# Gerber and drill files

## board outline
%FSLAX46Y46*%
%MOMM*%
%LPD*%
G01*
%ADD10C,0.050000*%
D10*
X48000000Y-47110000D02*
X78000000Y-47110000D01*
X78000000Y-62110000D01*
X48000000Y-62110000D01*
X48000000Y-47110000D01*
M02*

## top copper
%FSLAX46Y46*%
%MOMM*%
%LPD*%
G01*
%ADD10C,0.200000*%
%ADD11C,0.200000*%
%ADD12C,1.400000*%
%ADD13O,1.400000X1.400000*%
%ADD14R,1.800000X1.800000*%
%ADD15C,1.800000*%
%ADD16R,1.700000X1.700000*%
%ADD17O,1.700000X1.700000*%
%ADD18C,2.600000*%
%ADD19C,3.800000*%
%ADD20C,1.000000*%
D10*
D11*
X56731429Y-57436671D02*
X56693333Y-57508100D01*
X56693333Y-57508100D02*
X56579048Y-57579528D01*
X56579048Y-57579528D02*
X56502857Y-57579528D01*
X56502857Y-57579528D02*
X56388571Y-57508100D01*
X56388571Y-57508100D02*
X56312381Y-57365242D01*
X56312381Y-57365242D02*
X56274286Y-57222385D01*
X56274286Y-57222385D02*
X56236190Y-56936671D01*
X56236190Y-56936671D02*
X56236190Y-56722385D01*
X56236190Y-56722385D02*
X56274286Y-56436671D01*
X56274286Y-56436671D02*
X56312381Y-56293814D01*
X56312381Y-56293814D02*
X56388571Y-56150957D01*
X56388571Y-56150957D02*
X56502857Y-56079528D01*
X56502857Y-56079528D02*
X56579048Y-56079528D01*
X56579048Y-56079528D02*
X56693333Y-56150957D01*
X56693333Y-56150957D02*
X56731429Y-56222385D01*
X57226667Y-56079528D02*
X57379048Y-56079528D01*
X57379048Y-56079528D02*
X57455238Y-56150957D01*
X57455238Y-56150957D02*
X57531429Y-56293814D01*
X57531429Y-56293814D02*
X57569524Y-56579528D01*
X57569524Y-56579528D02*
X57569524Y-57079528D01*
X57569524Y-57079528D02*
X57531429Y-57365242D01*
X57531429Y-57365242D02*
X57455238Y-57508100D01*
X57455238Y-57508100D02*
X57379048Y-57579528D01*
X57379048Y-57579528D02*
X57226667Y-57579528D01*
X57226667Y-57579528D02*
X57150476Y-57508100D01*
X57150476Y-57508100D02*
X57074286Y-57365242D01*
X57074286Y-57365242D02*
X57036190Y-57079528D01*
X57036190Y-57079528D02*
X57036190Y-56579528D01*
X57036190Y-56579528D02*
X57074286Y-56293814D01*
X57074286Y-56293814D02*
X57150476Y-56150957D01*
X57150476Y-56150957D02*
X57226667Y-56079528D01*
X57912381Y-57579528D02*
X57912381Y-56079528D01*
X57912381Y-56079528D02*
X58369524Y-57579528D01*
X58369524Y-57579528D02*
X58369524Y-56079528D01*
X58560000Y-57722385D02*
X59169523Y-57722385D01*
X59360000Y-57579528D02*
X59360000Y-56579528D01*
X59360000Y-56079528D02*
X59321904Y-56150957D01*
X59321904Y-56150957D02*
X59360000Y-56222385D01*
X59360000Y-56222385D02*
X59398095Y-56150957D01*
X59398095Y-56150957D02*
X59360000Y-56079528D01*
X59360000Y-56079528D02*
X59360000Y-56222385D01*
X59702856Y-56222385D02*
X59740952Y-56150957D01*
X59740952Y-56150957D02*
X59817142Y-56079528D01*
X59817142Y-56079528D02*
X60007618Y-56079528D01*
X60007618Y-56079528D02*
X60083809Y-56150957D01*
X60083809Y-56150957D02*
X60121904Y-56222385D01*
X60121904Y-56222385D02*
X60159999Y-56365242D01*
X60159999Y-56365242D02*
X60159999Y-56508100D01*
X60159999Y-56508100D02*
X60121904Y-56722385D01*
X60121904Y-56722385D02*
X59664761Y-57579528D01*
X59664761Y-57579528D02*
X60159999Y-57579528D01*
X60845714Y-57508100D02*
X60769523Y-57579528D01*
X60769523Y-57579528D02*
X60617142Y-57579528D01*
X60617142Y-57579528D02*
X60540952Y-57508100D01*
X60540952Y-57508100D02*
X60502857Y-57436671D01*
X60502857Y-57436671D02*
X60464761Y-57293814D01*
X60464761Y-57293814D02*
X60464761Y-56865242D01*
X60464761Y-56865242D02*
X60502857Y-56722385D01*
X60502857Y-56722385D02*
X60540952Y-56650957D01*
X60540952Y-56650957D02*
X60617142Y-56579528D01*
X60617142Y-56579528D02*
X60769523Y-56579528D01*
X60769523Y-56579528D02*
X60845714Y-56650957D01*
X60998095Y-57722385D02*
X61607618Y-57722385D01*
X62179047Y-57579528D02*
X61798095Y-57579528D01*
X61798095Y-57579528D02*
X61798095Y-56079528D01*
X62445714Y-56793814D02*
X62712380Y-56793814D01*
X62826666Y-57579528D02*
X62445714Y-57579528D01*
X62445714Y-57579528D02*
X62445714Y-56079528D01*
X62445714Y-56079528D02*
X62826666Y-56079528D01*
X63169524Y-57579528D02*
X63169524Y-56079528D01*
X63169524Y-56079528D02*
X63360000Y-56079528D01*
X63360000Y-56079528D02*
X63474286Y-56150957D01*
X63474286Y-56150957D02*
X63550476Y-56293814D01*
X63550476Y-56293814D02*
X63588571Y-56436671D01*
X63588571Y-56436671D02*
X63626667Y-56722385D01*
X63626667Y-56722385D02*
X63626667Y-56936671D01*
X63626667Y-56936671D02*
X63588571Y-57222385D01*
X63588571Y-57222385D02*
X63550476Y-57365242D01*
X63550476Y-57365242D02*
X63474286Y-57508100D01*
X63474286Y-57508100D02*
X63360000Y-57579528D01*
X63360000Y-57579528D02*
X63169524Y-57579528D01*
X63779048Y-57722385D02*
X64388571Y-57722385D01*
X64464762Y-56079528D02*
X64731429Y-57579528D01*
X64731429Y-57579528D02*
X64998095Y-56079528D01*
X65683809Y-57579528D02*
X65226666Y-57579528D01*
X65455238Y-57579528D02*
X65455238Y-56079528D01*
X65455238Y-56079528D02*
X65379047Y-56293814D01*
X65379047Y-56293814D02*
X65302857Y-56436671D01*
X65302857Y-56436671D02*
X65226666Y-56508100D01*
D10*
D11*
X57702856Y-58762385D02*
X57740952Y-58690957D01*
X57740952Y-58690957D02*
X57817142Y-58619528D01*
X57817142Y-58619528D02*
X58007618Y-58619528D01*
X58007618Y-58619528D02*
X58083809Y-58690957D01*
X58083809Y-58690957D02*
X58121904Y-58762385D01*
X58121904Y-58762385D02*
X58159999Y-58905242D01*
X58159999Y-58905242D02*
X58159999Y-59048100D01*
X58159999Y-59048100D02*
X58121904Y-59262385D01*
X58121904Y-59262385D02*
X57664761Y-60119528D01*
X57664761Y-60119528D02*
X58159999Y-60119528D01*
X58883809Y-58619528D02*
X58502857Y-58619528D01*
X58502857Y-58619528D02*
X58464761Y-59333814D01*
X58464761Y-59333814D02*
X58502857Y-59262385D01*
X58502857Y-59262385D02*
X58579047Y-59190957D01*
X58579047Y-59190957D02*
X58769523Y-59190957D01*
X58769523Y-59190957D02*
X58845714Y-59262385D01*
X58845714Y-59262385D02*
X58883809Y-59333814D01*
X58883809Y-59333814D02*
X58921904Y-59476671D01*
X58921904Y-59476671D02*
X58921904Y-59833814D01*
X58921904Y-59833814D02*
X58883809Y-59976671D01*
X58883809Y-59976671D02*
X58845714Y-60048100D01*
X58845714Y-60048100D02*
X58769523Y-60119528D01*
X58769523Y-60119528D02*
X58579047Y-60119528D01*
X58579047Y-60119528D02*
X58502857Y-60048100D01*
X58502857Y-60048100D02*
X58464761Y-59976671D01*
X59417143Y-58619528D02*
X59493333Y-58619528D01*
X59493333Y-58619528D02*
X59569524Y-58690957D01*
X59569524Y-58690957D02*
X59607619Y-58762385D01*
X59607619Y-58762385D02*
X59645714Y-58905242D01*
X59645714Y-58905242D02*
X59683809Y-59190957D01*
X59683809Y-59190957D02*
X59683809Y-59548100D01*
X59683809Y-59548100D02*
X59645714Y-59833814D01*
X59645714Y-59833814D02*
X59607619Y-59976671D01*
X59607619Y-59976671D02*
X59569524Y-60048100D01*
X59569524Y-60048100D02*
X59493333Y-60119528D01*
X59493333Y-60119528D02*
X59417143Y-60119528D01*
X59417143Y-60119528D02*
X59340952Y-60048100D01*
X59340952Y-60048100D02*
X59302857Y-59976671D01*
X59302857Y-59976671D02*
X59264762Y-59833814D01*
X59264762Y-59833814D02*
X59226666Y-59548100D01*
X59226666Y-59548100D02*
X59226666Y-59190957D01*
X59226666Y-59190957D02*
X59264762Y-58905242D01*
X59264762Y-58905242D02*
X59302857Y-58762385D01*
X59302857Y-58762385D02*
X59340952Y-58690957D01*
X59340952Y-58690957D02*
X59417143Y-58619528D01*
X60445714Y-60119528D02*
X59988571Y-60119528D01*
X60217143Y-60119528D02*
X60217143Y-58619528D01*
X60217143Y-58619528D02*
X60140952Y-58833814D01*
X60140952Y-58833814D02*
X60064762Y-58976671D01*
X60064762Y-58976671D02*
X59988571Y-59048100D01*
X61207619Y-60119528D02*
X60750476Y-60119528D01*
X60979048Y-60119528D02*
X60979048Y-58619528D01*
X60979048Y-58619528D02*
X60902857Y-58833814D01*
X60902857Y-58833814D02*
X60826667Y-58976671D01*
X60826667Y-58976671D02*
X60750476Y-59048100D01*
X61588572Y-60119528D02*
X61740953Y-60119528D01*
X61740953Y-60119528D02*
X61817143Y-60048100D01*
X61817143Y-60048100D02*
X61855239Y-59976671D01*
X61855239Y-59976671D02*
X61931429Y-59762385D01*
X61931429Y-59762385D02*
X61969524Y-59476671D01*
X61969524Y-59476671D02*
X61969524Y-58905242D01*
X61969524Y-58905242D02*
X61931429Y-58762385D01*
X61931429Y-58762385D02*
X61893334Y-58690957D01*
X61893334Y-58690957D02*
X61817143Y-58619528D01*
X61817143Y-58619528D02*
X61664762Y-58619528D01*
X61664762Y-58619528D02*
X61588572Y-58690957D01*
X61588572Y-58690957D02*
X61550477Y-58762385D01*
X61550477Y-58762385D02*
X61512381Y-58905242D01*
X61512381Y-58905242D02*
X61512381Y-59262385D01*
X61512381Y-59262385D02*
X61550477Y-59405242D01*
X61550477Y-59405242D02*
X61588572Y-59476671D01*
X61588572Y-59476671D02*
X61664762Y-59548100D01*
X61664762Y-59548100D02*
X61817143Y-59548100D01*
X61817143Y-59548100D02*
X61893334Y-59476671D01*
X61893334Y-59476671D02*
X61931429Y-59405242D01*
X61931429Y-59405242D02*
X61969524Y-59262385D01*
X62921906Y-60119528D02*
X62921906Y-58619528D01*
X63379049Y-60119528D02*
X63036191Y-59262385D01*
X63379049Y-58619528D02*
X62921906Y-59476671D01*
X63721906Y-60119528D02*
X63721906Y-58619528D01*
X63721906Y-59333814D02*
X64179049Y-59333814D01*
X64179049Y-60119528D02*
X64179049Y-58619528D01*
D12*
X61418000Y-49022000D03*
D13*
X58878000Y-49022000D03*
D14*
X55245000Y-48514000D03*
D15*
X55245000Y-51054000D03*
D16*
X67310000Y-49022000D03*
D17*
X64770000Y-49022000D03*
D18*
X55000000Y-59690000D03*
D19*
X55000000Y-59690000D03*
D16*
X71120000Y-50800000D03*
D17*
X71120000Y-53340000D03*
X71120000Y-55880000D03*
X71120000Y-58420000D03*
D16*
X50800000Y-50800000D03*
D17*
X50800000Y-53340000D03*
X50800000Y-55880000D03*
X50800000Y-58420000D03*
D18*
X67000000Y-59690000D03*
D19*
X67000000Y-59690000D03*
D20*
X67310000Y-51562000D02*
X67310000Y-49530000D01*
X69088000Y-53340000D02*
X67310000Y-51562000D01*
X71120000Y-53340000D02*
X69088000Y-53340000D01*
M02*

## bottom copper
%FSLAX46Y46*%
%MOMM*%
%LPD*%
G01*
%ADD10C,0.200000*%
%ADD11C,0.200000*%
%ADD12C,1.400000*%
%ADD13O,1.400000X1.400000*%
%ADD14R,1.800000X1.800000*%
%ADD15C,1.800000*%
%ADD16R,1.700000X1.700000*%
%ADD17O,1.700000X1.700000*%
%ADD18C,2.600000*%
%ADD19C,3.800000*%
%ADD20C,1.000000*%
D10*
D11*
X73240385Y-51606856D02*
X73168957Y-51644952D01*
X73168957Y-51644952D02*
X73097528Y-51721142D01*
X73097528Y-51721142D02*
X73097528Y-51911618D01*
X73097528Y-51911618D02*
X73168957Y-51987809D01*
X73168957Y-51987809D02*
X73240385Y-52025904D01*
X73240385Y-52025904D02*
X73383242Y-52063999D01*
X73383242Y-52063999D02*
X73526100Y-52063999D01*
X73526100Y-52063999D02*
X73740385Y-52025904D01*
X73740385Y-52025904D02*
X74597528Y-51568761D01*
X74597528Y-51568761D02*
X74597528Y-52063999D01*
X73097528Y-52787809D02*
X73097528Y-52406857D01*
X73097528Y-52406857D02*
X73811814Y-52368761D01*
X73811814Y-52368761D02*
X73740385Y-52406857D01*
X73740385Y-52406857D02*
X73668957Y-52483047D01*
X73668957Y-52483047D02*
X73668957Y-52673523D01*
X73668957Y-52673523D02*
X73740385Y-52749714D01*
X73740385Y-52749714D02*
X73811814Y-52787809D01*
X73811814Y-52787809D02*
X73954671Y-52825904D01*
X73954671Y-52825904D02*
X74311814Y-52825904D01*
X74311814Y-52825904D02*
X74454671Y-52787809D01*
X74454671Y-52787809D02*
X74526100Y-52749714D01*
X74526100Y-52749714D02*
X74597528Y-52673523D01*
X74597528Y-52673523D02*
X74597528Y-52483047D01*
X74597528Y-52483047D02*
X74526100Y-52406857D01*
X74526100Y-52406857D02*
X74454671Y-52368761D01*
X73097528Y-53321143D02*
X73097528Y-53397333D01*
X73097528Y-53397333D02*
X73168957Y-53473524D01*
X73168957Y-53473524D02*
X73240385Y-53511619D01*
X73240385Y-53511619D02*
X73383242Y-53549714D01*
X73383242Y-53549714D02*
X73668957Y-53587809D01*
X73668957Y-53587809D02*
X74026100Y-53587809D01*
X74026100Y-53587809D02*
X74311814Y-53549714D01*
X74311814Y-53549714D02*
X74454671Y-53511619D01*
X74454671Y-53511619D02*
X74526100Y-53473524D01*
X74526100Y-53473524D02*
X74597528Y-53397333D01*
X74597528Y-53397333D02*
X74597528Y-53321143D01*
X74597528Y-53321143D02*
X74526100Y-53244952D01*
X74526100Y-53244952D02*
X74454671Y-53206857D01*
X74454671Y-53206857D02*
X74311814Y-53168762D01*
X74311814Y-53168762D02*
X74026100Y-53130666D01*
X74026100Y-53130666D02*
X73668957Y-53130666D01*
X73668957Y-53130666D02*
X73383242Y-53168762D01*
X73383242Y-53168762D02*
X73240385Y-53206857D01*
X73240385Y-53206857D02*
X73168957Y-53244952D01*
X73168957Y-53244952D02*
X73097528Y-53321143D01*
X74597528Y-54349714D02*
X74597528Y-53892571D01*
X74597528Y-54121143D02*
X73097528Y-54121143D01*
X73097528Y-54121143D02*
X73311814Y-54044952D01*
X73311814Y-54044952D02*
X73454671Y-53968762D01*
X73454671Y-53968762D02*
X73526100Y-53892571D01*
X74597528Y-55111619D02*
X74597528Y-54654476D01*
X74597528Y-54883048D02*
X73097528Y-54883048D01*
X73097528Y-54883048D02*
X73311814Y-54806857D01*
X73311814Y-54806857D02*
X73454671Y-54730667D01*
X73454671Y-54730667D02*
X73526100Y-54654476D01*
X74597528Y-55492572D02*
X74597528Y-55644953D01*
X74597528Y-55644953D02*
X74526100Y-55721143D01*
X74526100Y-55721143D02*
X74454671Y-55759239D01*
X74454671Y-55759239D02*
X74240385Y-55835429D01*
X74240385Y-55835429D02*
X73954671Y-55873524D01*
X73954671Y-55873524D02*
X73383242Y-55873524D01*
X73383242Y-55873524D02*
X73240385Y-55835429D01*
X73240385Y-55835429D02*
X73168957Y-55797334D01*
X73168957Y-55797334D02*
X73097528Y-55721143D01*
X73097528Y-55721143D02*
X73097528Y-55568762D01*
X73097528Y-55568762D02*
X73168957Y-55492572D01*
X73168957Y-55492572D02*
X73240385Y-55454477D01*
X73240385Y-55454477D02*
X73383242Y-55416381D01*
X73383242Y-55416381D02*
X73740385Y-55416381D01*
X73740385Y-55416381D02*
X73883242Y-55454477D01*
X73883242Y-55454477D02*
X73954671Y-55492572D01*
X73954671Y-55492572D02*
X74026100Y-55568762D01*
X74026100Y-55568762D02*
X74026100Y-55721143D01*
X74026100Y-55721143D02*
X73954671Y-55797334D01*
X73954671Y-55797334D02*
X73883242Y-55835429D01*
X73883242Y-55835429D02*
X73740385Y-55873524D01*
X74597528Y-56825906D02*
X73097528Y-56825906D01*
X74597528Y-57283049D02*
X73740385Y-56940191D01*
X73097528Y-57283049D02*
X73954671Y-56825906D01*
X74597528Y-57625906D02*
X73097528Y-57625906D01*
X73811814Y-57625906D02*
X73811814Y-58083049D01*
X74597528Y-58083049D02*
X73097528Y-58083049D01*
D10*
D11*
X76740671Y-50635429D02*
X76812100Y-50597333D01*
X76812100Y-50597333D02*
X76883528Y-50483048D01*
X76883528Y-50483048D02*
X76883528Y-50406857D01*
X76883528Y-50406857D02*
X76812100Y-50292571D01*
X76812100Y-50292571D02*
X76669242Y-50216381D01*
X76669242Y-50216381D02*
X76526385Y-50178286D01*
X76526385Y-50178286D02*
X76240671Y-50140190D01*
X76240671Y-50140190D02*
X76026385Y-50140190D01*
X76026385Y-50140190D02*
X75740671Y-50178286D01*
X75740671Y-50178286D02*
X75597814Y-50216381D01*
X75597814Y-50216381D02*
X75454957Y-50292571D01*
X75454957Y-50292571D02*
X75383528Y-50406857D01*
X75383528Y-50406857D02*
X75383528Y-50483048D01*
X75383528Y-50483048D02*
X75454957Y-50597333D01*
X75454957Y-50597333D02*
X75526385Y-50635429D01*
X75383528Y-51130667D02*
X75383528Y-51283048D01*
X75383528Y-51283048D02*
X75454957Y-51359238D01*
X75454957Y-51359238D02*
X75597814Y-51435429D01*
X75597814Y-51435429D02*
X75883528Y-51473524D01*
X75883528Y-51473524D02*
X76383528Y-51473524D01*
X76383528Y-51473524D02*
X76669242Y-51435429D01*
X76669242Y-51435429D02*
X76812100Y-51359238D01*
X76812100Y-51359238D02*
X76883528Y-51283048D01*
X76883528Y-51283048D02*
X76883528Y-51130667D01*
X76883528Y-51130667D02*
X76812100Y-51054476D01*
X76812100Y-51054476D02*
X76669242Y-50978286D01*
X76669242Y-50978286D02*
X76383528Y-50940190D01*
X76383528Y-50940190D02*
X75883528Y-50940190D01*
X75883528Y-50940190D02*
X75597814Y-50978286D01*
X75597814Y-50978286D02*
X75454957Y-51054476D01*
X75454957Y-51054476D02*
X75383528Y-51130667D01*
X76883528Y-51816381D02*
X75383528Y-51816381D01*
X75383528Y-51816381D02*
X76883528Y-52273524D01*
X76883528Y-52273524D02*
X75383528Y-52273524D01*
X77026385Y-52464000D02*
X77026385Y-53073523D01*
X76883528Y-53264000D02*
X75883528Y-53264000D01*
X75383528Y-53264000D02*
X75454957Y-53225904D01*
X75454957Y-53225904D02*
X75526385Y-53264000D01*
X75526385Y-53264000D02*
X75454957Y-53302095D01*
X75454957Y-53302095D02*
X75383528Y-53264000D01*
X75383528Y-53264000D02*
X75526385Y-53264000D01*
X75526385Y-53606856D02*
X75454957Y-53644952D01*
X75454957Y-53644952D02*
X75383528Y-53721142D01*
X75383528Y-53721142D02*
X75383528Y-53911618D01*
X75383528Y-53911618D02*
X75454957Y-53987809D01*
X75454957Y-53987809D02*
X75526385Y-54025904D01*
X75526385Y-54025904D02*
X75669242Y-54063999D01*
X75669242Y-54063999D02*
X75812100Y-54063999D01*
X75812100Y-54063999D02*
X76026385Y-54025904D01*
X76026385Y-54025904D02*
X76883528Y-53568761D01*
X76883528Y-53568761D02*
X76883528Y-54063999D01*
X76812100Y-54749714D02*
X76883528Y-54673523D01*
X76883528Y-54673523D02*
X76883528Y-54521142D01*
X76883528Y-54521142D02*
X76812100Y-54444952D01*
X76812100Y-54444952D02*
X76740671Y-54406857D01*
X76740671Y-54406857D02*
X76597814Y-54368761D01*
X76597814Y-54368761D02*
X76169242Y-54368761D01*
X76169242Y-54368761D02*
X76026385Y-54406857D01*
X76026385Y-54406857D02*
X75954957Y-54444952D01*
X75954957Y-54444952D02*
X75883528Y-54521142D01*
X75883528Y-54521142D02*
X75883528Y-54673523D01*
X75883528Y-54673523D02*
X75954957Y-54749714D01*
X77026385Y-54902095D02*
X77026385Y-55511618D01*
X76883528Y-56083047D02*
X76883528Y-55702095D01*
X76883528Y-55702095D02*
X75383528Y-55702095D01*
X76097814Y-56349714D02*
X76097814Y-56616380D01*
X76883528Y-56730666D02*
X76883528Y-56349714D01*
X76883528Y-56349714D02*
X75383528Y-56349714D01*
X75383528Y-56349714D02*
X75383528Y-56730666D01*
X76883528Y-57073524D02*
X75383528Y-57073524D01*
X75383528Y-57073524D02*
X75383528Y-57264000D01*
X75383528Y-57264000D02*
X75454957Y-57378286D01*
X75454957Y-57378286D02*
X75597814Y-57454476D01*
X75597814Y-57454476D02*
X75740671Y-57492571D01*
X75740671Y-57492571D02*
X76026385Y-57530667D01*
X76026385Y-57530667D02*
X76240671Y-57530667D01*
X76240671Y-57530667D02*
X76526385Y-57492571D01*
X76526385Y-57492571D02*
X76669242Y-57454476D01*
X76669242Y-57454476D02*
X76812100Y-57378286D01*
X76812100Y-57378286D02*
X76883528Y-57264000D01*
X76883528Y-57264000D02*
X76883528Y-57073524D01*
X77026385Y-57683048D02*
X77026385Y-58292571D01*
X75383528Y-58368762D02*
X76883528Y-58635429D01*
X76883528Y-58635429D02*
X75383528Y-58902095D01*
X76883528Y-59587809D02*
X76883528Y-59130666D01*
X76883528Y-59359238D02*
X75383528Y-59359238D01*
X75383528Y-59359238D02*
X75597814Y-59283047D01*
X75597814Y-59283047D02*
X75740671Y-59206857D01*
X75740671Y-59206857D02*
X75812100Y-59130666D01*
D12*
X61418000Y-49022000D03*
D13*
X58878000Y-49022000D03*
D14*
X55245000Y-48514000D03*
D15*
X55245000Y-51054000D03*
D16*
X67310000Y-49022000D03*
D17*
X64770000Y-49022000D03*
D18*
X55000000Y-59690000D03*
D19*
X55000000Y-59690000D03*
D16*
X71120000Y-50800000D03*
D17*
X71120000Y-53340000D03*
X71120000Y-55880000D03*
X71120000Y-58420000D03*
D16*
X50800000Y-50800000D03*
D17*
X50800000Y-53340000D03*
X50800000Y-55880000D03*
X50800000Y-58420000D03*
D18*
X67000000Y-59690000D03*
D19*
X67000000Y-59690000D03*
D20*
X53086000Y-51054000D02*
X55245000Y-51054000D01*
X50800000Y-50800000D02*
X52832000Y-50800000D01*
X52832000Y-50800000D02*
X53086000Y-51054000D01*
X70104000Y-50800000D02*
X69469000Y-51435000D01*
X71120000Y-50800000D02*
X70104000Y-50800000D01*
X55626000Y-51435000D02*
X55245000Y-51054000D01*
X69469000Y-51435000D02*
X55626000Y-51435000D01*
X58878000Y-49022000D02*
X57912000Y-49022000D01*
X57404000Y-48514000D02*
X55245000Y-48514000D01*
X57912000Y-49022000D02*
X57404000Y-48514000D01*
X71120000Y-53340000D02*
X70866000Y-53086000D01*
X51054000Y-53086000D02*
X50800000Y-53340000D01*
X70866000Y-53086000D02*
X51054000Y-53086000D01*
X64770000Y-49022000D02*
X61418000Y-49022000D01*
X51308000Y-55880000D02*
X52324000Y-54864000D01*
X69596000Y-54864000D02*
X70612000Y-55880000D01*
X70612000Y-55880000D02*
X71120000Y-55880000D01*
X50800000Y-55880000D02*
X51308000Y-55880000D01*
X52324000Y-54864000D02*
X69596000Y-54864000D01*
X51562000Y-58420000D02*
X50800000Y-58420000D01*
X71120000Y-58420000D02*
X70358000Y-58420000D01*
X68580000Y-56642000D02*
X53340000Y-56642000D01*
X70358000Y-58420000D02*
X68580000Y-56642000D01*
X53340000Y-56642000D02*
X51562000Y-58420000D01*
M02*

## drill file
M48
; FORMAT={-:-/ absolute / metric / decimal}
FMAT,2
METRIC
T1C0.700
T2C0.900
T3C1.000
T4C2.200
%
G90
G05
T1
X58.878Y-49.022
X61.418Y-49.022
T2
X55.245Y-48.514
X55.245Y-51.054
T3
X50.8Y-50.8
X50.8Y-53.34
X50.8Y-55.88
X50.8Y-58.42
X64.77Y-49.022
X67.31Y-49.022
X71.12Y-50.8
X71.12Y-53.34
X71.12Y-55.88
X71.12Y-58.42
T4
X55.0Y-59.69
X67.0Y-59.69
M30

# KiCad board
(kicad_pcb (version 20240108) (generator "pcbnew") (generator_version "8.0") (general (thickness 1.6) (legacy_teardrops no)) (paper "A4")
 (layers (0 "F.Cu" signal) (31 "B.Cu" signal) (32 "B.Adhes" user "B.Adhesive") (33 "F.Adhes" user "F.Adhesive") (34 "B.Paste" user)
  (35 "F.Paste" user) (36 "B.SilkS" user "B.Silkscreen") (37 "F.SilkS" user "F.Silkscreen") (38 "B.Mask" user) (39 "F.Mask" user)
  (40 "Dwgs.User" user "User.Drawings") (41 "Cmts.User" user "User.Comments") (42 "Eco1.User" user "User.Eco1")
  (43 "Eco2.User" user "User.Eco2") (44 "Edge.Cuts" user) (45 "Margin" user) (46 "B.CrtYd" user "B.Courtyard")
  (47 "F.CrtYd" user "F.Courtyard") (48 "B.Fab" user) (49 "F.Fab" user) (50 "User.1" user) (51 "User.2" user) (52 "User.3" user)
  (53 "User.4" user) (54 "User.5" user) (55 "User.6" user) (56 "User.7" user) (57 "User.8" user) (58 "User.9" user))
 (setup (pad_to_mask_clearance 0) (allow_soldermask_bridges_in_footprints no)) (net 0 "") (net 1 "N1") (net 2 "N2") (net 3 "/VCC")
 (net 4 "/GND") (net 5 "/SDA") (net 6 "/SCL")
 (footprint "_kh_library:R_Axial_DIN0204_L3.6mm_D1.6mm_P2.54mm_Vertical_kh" (layer "F.Cu") (at 61.418 49.022 180)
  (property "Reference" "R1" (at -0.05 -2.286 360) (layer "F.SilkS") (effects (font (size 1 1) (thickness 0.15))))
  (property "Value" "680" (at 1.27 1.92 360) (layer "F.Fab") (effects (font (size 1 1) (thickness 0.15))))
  (pad "1" thru_hole circle (at 0 0 180) (size 1.4 1.4) (drill 0.7) (layers "*.Cu" "*.Mask") (remove_unused_layers no) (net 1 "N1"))
  (pad "2" thru_hole oval (at 2.54 0 180) (size 1.4 1.4) (drill 0.7) (layers "*.Cu" "*.Mask") (remove_unused_layers no) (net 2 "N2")))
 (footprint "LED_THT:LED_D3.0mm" (layer "F.Cu") (at 55.245 48.514 -90)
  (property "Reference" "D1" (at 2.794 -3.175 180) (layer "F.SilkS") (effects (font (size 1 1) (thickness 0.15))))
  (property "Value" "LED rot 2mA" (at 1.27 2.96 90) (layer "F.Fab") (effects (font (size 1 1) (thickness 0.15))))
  (pad "1" thru_hole rect (at 0 0 270) (size 1.8 1.8) (drill 0.9) (layers "*.Cu" "*.Mask") (remove_unused_layers no) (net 2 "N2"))
  (pad "2" thru_hole circle (at 2.54 0 270) (size 1.8 1.8) (drill 0.9) (layers "*.Cu" "*.Mask") (remove_unused_layers no) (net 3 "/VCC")))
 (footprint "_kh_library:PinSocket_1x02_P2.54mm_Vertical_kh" (layer "F.Cu") (at 67.31 49.022 -90)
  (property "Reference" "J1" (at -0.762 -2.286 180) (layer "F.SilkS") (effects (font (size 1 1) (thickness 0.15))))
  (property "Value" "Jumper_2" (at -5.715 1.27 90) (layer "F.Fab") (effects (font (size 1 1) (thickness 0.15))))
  (pad "1" thru_hole rect (at 0 0 270) (size 1.7 1.7) (drill 1) (layers "*.Cu" "*.Mask") (remove_unused_layers no) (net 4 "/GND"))
  (pad "2" thru_hole oval (at 0 2.54 270) (size 1.7 1.7) (drill 1) (layers "*.Cu" "*.Mask") (remove_unused_layers no) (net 1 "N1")))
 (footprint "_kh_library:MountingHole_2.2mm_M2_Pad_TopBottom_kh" (layer "F.Cu") (at 55 59.69)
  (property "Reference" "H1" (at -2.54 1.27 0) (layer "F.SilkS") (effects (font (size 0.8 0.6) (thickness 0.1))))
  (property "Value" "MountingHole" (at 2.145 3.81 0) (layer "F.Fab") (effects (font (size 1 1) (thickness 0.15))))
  (pad "1" thru_hole circle (at 0 0) (size 2.6 2.6) (drill 2.2) (layers "*.Cu" "*.Mask") (remove_unused_layers no))
  (pad "1" connect circle (at 0 0) (size 3.8 3.8) (layers "F.Cu" "F.Mask"))
  (pad "1" connect circle (at 0 0) (size 3.8 3.8) (layers "B.Cu" "B.Mask")))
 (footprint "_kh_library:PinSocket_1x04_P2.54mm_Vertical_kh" (layer "F.Cu") (at 71.12 50.8)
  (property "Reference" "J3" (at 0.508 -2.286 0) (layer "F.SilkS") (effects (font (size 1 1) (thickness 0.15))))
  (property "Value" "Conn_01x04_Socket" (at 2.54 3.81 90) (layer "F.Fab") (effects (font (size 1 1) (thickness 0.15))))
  (pad "1" thru_hole rect (at 0 0) (size 1.7 1.7) (drill 1) (layers "*.Cu" "*.Mask") (remove_unused_layers no) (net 3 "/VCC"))
  (pad "2" thru_hole oval (at 0 2.54) (size 1.7 1.7) (drill 1) (layers "*.Cu" "*.Mask") (remove_unused_layers no) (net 4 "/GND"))
  (pad "3" thru_hole oval (at 0 5.08) (size 1.7 1.7) (drill 1) (layers "*.Cu" "*.Mask") (remove_unused_layers no) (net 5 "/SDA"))
  (pad "4" thru_hole oval (at 0 7.62) (size 1.7 1.7) (drill 1) (layers "*.Cu" "*.Mask") (remove_unused_layers no) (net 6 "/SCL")))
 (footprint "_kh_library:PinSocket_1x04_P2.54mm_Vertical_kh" (layer "F.Cu") (at 50.8 50.8)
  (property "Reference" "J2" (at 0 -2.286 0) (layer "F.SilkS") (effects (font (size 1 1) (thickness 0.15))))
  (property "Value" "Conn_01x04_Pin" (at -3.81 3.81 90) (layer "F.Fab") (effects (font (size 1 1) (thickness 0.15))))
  (pad "1" thru_hole rect (at 0 0) (size 1.7 1.7) (drill 1) (layers "*.Cu" "*.Mask") (remove_unused_layers no) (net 3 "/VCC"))
  (pad "2" thru_hole oval (at 0 2.54) (size 1.7 1.7) (drill 1) (layers "*.Cu" "*.Mask") (remove_unused_layers no) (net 4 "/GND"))
  (pad "3" thru_hole oval (at 0 5.08) (size 1.7 1.7) (drill 1) (layers "*.Cu" "*.Mask") (remove_unused_layers no) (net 5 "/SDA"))
  (pad "4" thru_hole oval (at 0 7.62) (size 1.7 1.7) (drill 1) (layers "*.Cu" "*.Mask") (remove_unused_layers no) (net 6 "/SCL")))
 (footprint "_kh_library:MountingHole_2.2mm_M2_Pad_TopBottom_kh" (layer "F.Cu") (at 67 59.69)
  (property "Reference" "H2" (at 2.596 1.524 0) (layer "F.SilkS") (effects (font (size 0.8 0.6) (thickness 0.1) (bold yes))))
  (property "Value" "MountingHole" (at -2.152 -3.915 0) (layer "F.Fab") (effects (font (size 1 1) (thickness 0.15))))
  (pad "1" thru_hole circle (at 0 0) (size 2.6 2.6) (drill 2.2) (layers "*.Cu" "*.Mask") (remove_unused_layers no))
  (pad "1" connect circle (at 0 0) (size 3.8 3.8) (layers "F.Cu" "F.Mask"))
  (pad "1" connect circle (at 0 0) (size 3.8 3.8) (layers "B.Cu" "B.Mask")))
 (gr_rect (start 48 47.11) (end 78 62.11) (stroke (width 0.05) (type default)) (fill none) (layer "Edge.Cuts"))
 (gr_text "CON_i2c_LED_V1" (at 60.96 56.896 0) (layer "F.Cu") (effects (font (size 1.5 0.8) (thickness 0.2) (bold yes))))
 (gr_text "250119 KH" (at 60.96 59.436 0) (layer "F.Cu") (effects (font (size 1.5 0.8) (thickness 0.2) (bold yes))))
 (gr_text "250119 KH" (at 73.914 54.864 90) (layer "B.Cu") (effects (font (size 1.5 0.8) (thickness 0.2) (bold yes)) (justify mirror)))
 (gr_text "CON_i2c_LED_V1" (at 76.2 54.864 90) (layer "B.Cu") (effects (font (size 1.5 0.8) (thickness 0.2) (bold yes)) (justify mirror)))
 (segment (start 53.086 51.054) (end 55.245 51.054) (width 1) (layer "B.Cu") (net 3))
 (segment (start 50.8 50.8) (end 52.832 50.8) (width 1) (layer "B.Cu") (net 3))
 (segment (start 52.832 50.8) (end 53.086 51.054) (width 1) (layer "B.Cu") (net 3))
 (segment (start 70.104 50.8) (end 69.469 51.435) (width 1) (layer "B.Cu") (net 3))
 (segment (start 71.12 50.8) (end 70.104 50.8) (width 1) (layer "B.Cu") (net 3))
 (segment (start 55.626 51.435) (end 55.245 51.054) (width 1) (layer "B.Cu") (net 3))
 (segment (start 69.469 51.435) (end 55.626 51.435) (width 1) (layer "B.Cu") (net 3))
 (segment (start 58.878 49.022) (end 57.912 49.022) (width 1) (layer "B.Cu") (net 2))
 (segment (start 57.404 48.514) (end 55.245 48.514) (width 1) (layer "B.Cu") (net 2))
 (segment (start 57.912 49.022) (end 57.404 48.514) (width 1) (layer "B.Cu") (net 2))
 (segment (start 67.31 51.562) (end 67.31 49.53) (width 1) (layer "F.Cu") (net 4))
 (segment (start 69.088 53.34) (end 67.31 51.562) (width 1) (layer "F.Cu") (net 4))
 (segment (start 71.12 53.34) (end 69.088 53.34) (width 1) (layer "F.Cu") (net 4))
 (segment (start 71.12 53.34) (end 70.866 53.086) (width 1) (layer "B.Cu") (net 4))
 (segment (start 51.054 53.086) (end 50.8 53.34) (width 1) (layer "B.Cu") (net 4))
 (segment (start 70.866 53.086) (end 51.054 53.086) (width 1) (layer "B.Cu") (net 4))
 (segment (start 64.77 49.022) (end 61.418 49.022) (width 1) (layer "B.Cu") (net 1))
 (segment (start 51.308 55.88) (end 52.324 54.864) (width 1) (layer "B.Cu") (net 5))
 (segment (start 69.596 54.864) (end 70.612 55.88) (width 1) (layer "B.Cu") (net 5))
 (segment (start 70.612 55.88) (end 71.12 55.88) (width 1) (layer "B.Cu") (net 5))
 (segment (start 50.8 55.88) (end 51.308 55.88) (width 1) (layer "B.Cu") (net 5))
 (segment (start 52.324 54.864) (end 69.596 54.864) (width 1) (layer "B.Cu") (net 5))
 (segment (start 51.562 58.42) (end 50.8 58.42) (width 1) (layer "B.Cu") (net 6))
 (segment (start 71.12 58.42) (end 70.358 58.42) (width 1) (layer "B.Cu") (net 6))
 (segment (start 68.58 56.642) (end 53.34 56.642) (width 1) (layer "B.Cu") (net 6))
 (segment (start 70.358 58.42) (end 68.58 56.642) (width 1) (layer "B.Cu") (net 6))
 (segment (start 53.34 56.642) (end 51.562 58.42) (width 1) (layer "B.Cu") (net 6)))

